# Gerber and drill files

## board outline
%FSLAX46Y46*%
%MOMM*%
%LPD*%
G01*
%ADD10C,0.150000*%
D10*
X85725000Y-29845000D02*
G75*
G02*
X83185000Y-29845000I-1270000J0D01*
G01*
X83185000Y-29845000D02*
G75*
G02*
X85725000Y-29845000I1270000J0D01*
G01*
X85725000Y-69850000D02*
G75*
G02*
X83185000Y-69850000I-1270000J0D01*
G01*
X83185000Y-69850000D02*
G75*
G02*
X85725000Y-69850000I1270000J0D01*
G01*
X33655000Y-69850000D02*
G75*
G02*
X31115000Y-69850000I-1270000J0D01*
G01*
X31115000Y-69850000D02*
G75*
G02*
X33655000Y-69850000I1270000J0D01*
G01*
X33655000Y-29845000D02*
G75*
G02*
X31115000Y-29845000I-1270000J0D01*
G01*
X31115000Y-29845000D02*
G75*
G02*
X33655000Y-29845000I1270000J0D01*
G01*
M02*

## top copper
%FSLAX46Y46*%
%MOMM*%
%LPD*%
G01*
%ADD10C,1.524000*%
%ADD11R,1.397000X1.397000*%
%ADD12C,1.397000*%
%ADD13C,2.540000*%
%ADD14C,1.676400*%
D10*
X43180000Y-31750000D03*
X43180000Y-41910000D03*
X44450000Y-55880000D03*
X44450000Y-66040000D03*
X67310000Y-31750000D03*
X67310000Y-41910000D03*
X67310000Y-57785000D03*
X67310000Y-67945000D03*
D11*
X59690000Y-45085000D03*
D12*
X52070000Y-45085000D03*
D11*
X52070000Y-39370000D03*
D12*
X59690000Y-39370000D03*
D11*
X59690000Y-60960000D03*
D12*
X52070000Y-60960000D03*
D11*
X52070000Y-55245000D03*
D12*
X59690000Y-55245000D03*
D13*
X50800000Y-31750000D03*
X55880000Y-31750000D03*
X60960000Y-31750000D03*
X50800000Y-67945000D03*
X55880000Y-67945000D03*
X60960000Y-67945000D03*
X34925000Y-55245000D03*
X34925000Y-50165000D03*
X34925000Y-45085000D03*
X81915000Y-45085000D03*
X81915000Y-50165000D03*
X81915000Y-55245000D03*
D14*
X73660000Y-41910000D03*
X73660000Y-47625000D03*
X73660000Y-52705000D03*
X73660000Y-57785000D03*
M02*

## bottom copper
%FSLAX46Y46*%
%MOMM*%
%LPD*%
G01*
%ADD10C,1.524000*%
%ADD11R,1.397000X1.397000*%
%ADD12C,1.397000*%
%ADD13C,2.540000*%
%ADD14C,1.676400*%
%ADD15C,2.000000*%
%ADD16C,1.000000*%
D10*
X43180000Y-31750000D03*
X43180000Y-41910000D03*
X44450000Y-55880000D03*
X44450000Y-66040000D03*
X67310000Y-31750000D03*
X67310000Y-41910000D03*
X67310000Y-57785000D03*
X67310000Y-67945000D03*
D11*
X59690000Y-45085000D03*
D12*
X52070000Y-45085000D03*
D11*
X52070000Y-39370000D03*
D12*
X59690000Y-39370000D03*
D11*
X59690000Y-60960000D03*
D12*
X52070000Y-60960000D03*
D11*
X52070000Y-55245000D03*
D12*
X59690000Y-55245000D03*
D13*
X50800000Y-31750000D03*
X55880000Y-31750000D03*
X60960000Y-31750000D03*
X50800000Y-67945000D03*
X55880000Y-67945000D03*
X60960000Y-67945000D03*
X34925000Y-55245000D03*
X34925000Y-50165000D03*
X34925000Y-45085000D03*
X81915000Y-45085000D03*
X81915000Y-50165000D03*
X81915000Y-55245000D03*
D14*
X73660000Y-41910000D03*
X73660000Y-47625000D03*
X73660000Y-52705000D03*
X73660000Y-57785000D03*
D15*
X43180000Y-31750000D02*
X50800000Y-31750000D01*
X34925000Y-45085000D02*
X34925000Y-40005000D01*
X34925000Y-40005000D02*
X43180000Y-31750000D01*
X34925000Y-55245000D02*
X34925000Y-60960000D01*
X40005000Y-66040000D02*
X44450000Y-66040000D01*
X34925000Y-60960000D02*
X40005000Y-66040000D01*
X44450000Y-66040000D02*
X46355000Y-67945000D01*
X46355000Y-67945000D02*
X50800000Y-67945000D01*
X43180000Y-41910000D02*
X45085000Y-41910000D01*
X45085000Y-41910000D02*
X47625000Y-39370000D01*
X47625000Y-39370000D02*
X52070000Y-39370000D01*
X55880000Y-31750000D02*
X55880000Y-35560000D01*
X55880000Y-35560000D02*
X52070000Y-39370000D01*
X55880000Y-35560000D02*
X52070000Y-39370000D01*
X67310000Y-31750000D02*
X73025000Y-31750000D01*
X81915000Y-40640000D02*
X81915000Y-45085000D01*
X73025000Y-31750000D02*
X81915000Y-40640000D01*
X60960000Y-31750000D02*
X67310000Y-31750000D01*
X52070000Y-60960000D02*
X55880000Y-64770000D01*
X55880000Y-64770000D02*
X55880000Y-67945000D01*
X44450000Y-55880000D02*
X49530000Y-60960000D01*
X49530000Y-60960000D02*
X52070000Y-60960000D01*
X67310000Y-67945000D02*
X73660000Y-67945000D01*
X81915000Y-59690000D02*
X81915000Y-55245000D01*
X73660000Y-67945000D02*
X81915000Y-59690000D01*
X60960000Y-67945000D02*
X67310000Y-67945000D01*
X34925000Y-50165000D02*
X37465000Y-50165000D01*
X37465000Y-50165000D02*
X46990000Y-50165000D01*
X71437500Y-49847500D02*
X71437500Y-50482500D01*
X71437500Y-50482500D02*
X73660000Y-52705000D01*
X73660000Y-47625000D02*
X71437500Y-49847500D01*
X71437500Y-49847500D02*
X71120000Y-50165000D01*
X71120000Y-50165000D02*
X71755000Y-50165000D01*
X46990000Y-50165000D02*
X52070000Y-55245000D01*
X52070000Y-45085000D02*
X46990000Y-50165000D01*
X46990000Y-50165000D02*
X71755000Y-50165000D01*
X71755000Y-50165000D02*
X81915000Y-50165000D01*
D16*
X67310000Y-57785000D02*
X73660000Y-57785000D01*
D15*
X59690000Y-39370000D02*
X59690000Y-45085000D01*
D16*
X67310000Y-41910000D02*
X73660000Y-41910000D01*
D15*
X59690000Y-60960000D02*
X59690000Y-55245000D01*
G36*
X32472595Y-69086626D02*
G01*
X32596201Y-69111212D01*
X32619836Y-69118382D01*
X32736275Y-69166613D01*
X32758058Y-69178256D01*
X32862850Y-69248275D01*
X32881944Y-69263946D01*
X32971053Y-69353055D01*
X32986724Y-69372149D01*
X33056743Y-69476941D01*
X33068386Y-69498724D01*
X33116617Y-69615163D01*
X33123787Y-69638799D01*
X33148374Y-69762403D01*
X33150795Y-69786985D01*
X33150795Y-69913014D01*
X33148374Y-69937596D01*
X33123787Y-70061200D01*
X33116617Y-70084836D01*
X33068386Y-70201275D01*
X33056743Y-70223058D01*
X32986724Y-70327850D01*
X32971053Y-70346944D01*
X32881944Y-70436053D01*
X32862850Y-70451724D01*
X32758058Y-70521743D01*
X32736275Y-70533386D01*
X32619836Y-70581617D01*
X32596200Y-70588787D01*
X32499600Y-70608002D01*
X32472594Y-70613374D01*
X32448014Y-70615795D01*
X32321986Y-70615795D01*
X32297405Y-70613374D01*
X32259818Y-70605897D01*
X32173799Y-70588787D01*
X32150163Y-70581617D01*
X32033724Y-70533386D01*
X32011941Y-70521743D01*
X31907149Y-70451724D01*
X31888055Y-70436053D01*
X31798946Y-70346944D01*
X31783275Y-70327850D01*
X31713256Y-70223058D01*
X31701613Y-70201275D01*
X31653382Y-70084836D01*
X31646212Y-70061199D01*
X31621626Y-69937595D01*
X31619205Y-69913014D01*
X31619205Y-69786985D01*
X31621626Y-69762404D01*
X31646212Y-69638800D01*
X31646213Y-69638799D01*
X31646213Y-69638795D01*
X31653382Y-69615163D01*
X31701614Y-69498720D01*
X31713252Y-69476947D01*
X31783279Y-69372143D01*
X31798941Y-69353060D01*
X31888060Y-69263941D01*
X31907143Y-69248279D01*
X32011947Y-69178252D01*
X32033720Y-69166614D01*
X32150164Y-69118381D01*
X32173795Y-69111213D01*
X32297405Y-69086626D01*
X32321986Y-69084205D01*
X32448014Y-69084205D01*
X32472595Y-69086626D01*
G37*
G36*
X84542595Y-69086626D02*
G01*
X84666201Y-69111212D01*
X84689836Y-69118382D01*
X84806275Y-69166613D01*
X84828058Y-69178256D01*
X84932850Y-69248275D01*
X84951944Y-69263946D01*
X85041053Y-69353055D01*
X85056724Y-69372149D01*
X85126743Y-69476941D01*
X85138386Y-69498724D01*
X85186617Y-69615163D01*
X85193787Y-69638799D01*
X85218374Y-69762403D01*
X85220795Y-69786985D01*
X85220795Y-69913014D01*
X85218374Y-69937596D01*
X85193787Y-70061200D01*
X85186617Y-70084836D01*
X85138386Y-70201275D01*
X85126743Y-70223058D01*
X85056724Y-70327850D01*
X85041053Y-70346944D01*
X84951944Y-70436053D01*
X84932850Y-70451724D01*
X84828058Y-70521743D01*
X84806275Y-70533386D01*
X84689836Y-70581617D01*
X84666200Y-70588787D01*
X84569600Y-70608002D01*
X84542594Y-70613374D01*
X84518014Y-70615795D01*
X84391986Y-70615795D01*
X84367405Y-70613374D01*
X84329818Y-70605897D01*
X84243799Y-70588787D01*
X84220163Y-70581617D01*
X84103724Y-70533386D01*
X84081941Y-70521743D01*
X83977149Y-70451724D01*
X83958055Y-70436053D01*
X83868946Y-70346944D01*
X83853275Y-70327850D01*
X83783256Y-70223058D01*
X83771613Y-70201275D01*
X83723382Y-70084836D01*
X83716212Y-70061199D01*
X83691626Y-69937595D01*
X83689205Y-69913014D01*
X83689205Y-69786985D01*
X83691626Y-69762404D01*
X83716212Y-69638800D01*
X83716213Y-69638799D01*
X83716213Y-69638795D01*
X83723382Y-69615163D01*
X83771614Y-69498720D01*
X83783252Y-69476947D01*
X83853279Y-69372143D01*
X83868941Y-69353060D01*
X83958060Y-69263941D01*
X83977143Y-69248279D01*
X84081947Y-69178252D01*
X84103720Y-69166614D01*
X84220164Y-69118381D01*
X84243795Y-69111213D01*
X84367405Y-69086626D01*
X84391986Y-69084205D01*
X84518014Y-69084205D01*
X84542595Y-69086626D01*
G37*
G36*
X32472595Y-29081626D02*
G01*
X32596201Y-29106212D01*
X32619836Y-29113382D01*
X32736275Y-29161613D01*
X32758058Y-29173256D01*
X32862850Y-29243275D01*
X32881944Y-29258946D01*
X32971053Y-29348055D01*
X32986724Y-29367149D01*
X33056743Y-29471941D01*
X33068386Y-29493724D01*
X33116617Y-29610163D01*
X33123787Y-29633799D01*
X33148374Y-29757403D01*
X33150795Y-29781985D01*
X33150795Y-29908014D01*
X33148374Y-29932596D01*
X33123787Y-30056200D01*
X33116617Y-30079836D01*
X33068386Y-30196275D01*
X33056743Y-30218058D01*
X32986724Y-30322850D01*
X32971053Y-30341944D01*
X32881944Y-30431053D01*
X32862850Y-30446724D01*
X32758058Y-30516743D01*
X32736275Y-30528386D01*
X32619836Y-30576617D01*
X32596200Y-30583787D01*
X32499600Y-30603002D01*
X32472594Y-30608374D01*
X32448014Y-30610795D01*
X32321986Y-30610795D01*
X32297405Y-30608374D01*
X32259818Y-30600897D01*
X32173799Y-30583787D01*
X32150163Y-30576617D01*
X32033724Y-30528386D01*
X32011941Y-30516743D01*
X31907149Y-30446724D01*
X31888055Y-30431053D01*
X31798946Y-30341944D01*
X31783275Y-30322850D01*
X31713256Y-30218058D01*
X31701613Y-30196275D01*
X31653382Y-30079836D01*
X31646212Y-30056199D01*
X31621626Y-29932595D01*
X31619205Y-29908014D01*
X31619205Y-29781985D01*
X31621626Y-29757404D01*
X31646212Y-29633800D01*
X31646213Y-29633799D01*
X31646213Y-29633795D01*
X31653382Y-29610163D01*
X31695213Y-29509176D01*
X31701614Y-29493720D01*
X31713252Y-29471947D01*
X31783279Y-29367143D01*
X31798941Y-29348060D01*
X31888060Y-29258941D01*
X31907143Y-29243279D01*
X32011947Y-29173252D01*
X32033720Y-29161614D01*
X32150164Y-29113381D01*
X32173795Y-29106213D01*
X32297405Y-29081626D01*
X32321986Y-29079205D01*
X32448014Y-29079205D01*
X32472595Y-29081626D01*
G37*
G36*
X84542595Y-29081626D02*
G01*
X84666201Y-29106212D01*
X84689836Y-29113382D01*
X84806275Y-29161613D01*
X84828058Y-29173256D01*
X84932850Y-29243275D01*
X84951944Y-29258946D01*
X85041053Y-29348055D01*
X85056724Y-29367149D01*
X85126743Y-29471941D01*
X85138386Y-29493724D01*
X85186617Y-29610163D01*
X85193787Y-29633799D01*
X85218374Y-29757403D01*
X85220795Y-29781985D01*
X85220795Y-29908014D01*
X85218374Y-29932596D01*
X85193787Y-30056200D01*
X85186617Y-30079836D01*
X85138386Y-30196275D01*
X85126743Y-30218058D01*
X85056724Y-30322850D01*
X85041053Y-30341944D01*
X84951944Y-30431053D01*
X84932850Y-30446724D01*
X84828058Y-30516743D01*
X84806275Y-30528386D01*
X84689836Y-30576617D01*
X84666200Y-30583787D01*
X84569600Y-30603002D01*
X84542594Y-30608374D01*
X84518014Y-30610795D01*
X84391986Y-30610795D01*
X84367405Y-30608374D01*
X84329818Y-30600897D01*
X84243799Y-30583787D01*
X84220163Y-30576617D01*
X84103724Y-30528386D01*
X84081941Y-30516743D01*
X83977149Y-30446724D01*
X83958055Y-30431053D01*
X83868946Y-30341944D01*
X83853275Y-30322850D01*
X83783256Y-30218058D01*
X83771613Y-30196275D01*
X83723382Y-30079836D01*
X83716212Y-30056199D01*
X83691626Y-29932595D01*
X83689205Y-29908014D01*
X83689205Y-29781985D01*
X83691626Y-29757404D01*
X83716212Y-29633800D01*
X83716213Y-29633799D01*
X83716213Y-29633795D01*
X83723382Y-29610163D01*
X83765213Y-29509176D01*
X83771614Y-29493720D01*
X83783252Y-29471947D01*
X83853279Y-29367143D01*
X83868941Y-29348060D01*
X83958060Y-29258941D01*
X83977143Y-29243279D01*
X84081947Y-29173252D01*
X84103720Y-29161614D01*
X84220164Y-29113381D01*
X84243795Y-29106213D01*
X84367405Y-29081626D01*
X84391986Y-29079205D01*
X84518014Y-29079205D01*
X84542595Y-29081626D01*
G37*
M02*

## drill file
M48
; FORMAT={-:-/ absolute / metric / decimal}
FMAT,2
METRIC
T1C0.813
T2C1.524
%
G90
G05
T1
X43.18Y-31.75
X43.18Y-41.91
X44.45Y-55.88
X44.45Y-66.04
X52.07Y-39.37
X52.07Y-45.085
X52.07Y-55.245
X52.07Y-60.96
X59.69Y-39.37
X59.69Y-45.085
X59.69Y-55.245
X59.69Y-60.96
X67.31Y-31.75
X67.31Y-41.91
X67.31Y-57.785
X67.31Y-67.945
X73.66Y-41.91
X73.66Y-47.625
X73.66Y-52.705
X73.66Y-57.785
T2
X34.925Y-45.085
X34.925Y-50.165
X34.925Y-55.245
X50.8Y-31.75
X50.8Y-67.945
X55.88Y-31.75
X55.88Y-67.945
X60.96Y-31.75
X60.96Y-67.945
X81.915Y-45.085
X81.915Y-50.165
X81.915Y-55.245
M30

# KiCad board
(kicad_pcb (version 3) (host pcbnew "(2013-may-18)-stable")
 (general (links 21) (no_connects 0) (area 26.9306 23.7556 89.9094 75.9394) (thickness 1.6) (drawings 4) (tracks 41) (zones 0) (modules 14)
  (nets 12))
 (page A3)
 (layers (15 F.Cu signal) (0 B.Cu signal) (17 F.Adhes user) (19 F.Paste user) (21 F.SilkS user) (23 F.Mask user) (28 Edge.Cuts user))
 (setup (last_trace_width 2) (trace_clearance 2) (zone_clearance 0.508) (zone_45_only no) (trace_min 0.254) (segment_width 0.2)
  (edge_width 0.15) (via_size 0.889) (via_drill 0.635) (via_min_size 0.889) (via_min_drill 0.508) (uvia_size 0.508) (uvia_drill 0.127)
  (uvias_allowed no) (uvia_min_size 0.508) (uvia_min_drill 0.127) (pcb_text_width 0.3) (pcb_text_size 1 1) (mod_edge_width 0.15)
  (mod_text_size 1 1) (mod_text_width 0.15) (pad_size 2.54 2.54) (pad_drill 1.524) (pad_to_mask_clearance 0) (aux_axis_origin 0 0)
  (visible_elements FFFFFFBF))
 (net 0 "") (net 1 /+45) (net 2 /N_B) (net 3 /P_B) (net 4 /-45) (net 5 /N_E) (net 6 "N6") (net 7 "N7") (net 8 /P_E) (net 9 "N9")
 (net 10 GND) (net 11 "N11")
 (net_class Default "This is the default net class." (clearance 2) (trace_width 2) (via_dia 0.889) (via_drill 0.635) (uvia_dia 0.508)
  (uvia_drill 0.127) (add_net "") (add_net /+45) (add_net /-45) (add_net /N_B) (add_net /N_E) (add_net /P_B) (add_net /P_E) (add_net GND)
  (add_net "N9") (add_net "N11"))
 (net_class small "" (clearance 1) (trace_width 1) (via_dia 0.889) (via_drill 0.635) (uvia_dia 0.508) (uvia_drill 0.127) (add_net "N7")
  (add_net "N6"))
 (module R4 (layer F.Cu) (at 43.18 36.83 270) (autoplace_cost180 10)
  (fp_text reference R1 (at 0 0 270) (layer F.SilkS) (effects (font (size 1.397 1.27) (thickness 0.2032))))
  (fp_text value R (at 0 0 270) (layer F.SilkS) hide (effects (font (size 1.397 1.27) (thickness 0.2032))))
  (pad 1 thru_hole circle (at -5.08 0 270) (size 1.524 1.524) (drill 0.8128) (layers *.Cu *.Mask F.SilkS) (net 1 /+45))
  (pad 2 thru_hole circle (at 5.08 0 270) (size 1.524 1.524) (drill 0.8128) (layers *.Cu *.Mask F.SilkS) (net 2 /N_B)))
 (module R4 (layer F.Cu) (at 44.45 60.96 270) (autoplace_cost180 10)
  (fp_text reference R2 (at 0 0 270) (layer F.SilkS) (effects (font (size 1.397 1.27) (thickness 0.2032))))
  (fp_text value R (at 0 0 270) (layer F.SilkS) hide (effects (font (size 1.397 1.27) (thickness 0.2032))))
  (pad 1 thru_hole circle (at -5.08 0 270) (size 1.524 1.524) (drill 0.8128) (layers *.Cu *.Mask F.SilkS) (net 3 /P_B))
  (pad 2 thru_hole circle (at 5.08 0 270) (size 1.524 1.524) (drill 0.8128) (layers *.Cu *.Mask F.SilkS) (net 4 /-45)))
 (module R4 (layer F.Cu) (at 67.31 36.83 270) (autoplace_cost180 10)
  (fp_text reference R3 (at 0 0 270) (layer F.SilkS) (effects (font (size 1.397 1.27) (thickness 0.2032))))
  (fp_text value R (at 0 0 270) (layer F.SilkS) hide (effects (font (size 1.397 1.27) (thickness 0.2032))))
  (pad 1 thru_hole circle (at -5.08 0 270) (size 1.524 1.524) (drill 0.8128) (layers *.Cu *.Mask F.SilkS) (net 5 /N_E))
  (pad 2 thru_hole circle (at 5.08 0 270) (size 1.524 1.524) (drill 0.8128) (layers *.Cu *.Mask F.SilkS) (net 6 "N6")))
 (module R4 (layer F.Cu) (at 67.31 62.865 270) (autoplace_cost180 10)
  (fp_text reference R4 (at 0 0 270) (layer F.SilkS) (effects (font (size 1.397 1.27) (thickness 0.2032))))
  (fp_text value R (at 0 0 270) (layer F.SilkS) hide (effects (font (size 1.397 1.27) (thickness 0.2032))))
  (pad 1 thru_hole circle (at -5.08 0 270) (size 1.524 1.524) (drill 0.8128) (layers *.Cu *.Mask F.SilkS) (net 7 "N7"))
  (pad 2 thru_hole circle (at 5.08 0 270) (size 1.524 1.524) (drill 0.8128) (layers *.Cu *.Mask F.SilkS) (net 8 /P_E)))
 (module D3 (layer F.Cu) (at 55.88 45.085)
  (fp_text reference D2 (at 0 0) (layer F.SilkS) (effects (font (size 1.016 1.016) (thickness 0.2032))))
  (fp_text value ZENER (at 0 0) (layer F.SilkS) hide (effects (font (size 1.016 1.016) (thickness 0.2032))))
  (pad 2 thru_hole rect (at 3.81 0) (size 1.397 1.397) (drill 0.8128) (layers *.Cu *.Mask F.SilkS) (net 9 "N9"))
  (pad 1 thru_hole circle (at -3.81 0) (size 1.397 1.397) (drill 0.8128) (layers *.Cu *.Mask F.SilkS) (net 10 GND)))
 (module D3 (layer F.Cu) (at 55.88 39.37 180)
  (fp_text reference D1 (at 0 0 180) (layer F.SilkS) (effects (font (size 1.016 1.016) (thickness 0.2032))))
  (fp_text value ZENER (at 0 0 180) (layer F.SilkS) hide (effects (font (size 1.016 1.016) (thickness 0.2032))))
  (pad 2 thru_hole rect (at 3.81 0 180) (size 1.397 1.397) (drill 0.8128) (layers *.Cu *.Mask F.SilkS) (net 2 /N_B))
  (pad 1 thru_hole circle (at -3.81 0 180) (size 1.397 1.397) (drill 0.8128) (layers *.Cu *.Mask F.SilkS) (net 9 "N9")))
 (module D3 (layer F.Cu) (at 55.88 60.96)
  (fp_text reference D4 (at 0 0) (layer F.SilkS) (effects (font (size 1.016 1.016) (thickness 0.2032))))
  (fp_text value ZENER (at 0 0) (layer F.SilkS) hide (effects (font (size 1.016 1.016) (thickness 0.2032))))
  (pad 2 thru_hole rect (at 3.81 0) (size 1.397 1.397) (drill 0.8128) (layers *.Cu *.Mask F.SilkS) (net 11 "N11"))
  (pad 1 thru_hole circle (at -3.81 0) (size 1.397 1.397) (drill 0.8128) (layers *.Cu *.Mask F.SilkS) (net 3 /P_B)))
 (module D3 (layer F.Cu) (at 55.88 55.245 180)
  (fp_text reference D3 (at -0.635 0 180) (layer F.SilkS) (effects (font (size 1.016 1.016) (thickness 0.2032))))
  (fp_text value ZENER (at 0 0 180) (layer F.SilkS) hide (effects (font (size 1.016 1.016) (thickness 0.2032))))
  (pad 2 thru_hole rect (at 3.81 0 180) (size 1.397 1.397) (drill 0.8128) (layers *.Cu *.Mask F.SilkS) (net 10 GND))
  (pad 1 thru_hole circle (at -3.81 0 180) (size 1.397 1.397) (drill 0.8128) (layers *.Cu *.Mask F.SilkS) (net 11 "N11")))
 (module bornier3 (layer F.Cu) (at 55.88 31.75)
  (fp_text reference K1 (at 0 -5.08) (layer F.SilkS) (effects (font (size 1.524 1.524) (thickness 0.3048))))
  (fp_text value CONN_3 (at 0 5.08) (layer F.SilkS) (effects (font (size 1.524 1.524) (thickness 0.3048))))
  (pad 1 thru_hole circle (at -5.08 0) (size 2.54 2.54) (drill 1.524) (layers *.Cu *.Mask F.SilkS) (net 1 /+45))
  (pad 2 thru_hole circle (at 0 0) (size 2.54 2.54) (drill 1.524) (layers *.Cu *.Mask F.SilkS) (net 2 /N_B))
  (pad 3 thru_hole circle (at 5.08 0) (size 2.54 2.54) (drill 1.524) (layers *.Cu *.Mask F.SilkS) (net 5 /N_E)))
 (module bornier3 (layer F.Cu) (at 55.88 67.945)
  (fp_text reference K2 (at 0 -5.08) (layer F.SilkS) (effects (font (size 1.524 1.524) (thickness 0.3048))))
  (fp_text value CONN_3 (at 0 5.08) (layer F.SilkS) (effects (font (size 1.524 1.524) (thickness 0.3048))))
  (pad 1 thru_hole circle (at -5.08 0) (size 2.54 2.54) (drill 1.524) (layers *.Cu *.Mask F.SilkS) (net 4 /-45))
  (pad 2 thru_hole circle (at 0 0) (size 2.54 2.54) (drill 1.524) (layers *.Cu *.Mask F.SilkS) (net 3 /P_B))
  (pad 3 thru_hole circle (at 5.08 0) (size 2.54 2.54) (drill 1.524) (layers *.Cu *.Mask F.SilkS) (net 8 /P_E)))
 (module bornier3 (layer F.Cu) (at 34.925 50.165 90)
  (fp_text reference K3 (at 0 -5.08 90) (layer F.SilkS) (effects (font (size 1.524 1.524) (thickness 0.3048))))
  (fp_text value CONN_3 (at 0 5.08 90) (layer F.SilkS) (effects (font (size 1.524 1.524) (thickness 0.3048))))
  (pad 1 thru_hole circle (at -5.08 0 90) (size 2.54 2.54) (drill 1.524) (layers *.Cu *.Mask F.SilkS) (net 4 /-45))
  (pad 2 thru_hole circle (at 0 0 90) (size 2.54 2.54) (drill 1.524) (layers *.Cu *.Mask F.SilkS) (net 10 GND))
  (pad 3 thru_hole circle (at 5.08 0 90) (size 2.54 2.54) (drill 1.524) (layers *.Cu *.Mask F.SilkS) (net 1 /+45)))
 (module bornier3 (layer F.Cu) (at 81.915 50.165 270)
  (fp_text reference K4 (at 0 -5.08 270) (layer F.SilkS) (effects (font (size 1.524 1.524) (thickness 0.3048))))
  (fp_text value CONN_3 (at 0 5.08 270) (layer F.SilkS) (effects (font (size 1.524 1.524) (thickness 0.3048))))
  (pad 1 thru_hole circle (at -5.08 0 270) (size 2.54 2.54) (drill 1.524) (layers *.Cu *.Mask F.SilkS) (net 5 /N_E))
  (pad 2 thru_hole circle (at 0 0 270) (size 2.54 2.54) (drill 1.524) (layers *.Cu *.Mask F.SilkS) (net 10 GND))
  (pad 3 thru_hole circle (at 5.08 0 270) (size 2.54 2.54) (drill 1.524) (layers *.Cu *.Mask F.SilkS) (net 8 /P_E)))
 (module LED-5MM (layer F.Cu) (at 73.66 43.18 270)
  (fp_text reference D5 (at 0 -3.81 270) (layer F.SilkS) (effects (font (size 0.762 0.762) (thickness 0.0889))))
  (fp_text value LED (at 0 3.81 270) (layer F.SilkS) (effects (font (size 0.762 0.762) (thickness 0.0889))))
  (pad 1 thru_hole circle (at -1.27 0 270) (size 1.6764 1.6764) (drill 0.8128) (layers *.Cu *.Mask F.SilkS) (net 6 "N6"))
  (pad 2 thru_hole circle (at 4.445 0 270) (size 1.6764 1.6764) (drill 0.8128) (layers *.Cu *.Mask F.SilkS) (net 10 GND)))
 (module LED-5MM (layer F.Cu) (at 73.66 56.515 270)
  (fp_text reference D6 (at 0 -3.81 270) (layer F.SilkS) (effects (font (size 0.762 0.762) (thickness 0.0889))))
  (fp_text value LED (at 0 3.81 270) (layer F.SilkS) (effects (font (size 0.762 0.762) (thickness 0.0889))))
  (pad 1 thru_hole circle (at -3.81 0 270) (size 1.6764 1.6764) (drill 0.8128) (layers *.Cu *.Mask F.SilkS) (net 10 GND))
  (pad 2 thru_hole circle (at 1.27 0 270) (size 1.6764 1.6764) (drill 0.8128) (layers *.Cu *.Mask F.SilkS) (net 7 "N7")))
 (gr_circle (center 84.455 29.845) (end 85.725 29.845) (layer Edge.Cuts) (width 0.15))
 (gr_circle (center 84.455 69.85) (end 85.725 69.85) (layer Edge.Cuts) (width 0.15))
 (gr_circle (center 32.385 69.85) (end 33.655 69.85) (layer Edge.Cuts) (width 0.15))
 (gr_circle (center 32.385 29.845) (end 33.655 29.845) (layer Edge.Cuts) (width 0.15))
 (segment (start 43.18 31.75) (end 50.8 31.75) (width 2) (layer B.Cu) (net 1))
 (segment (start 34.925 45.085) (end 34.925 40.005) (width 2) (layer B.Cu) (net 1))
 (segment (start 34.925 40.005) (end 43.18 31.75) (width 2) (layer B.Cu) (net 1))
 (segment (start 34.925 55.245) (end 34.925 60.96) (width 2) (layer B.Cu) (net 4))
 (segment (start 40.005 66.04) (end 44.45 66.04) (width 2) (layer B.Cu) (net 4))
 (segment (start 34.925 60.96) (end 40.005 66.04) (width 2) (layer B.Cu) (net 4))
 (segment (start 44.45 66.04) (end 46.355 67.945) (width 2) (layer B.Cu) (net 4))
 (segment (start 46.355 67.945) (end 50.8 67.945) (width 2) (layer B.Cu) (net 4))
 (segment (start 43.18 41.91) (end 45.085 41.91) (width 2) (layer B.Cu) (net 2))
 (segment (start 45.085 41.91) (end 47.625 39.37) (width 2) (layer B.Cu) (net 2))
 (segment (start 47.625 39.37) (end 52.07 39.37) (width 2) (layer B.Cu) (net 2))
 (segment (start 55.88 31.75) (end 55.88 35.56) (width 2) (layer B.Cu) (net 2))
 (segment (start 55.88 35.56) (end 52.07 39.37) (width 2) (layer B.Cu) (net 2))
 (segment (start 55.88 35.56) (end 52.07 39.37) (width 2) (layer B.Cu) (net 2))
 (segment (start 67.31 31.75) (end 73.025 31.75) (width 2) (layer B.Cu) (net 5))
 (segment (start 81.915 40.64) (end 81.915 45.085) (width 2) (layer B.Cu) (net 5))
 (segment (start 73.025 31.75) (end 81.915 40.64) (width 2) (layer B.Cu) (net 5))
 (segment (start 60.96 31.75) (end 67.31 31.75) (width 2) (layer B.Cu) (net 5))
 (segment (start 52.07 60.96) (end 55.88 64.77) (width 2) (layer B.Cu) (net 3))
 (segment (start 55.88 64.77) (end 55.88 67.945) (width 2) (layer B.Cu) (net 3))
 (segment (start 44.45 55.88) (end 49.53 60.96) (width 2) (layer B.Cu) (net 3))
 (segment (start 49.53 60.96) (end 52.07 60.96) (width 2) (layer B.Cu) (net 3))
 (segment (start 67.31 67.945) (end 73.66 67.945) (width 2) (layer B.Cu) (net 8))
 (segment (start 81.915 59.69) (end 81.915 55.245) (width 2) (layer B.Cu) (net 8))
 (segment (start 73.66 67.945) (end 81.915 59.69) (width 2) (layer B.Cu) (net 8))
 (segment (start 60.96 67.945) (end 67.31 67.945) (width 2) (layer B.Cu) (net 8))
 (segment (start 34.925 50.165) (end 37.465 50.165) (width 2) (layer B.Cu) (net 10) (status 400000))
 (segment (start 37.465 50.165) (end 46.99 50.165) (width 2) (layer B.Cu) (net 10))
 (segment (start 71.4375 49.8475) (end 71.4375 50.4825) (width 2) (layer B.Cu) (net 10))
 (segment (start 71.4375 50.4825) (end 73.66 52.705) (width 2) (layer B.Cu) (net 10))
 (segment (start 73.66 47.625) (end 71.4375 49.8475) (width 2) (layer B.Cu) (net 10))
 (segment (start 71.4375 49.8475) (end 71.12 50.165) (width 2) (layer B.Cu) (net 10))
 (segment (start 71.12 50.165) (end 71.755 50.165) (width 2) (layer B.Cu) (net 10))
 (segment (start 46.99 50.165) (end 52.07 55.245) (width 2) (layer B.Cu) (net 10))
 (segment (start 52.07 45.085) (end 46.99 50.165) (width 2) (layer B.Cu) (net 10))
 (segment (start 46.99 50.165) (end 71.755 50.165) (width 2) (layer B.Cu) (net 10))
 (segment (start 71.755 50.165) (end 81.915 50.165) (width 2) (layer B.Cu) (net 10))
 (segment (start 67.31 57.785) (end 73.66 57.785) (width 1) (layer B.Cu) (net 7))
 (segment (start 59.69 39.37) (end 59.69 45.085) (width 2) (layer B.Cu) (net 9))
 (segment (start 67.31 41.91) (end 73.66 41.91) (width 1) (layer B.Cu) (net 6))
 (segment (start 59.69 60.96) (end 59.69 55.245) (width 2) (layer B.Cu) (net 11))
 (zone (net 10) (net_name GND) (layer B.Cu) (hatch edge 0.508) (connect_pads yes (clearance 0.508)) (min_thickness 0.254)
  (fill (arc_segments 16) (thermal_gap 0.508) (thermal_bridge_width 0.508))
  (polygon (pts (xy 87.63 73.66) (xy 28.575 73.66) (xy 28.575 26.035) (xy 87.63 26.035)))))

